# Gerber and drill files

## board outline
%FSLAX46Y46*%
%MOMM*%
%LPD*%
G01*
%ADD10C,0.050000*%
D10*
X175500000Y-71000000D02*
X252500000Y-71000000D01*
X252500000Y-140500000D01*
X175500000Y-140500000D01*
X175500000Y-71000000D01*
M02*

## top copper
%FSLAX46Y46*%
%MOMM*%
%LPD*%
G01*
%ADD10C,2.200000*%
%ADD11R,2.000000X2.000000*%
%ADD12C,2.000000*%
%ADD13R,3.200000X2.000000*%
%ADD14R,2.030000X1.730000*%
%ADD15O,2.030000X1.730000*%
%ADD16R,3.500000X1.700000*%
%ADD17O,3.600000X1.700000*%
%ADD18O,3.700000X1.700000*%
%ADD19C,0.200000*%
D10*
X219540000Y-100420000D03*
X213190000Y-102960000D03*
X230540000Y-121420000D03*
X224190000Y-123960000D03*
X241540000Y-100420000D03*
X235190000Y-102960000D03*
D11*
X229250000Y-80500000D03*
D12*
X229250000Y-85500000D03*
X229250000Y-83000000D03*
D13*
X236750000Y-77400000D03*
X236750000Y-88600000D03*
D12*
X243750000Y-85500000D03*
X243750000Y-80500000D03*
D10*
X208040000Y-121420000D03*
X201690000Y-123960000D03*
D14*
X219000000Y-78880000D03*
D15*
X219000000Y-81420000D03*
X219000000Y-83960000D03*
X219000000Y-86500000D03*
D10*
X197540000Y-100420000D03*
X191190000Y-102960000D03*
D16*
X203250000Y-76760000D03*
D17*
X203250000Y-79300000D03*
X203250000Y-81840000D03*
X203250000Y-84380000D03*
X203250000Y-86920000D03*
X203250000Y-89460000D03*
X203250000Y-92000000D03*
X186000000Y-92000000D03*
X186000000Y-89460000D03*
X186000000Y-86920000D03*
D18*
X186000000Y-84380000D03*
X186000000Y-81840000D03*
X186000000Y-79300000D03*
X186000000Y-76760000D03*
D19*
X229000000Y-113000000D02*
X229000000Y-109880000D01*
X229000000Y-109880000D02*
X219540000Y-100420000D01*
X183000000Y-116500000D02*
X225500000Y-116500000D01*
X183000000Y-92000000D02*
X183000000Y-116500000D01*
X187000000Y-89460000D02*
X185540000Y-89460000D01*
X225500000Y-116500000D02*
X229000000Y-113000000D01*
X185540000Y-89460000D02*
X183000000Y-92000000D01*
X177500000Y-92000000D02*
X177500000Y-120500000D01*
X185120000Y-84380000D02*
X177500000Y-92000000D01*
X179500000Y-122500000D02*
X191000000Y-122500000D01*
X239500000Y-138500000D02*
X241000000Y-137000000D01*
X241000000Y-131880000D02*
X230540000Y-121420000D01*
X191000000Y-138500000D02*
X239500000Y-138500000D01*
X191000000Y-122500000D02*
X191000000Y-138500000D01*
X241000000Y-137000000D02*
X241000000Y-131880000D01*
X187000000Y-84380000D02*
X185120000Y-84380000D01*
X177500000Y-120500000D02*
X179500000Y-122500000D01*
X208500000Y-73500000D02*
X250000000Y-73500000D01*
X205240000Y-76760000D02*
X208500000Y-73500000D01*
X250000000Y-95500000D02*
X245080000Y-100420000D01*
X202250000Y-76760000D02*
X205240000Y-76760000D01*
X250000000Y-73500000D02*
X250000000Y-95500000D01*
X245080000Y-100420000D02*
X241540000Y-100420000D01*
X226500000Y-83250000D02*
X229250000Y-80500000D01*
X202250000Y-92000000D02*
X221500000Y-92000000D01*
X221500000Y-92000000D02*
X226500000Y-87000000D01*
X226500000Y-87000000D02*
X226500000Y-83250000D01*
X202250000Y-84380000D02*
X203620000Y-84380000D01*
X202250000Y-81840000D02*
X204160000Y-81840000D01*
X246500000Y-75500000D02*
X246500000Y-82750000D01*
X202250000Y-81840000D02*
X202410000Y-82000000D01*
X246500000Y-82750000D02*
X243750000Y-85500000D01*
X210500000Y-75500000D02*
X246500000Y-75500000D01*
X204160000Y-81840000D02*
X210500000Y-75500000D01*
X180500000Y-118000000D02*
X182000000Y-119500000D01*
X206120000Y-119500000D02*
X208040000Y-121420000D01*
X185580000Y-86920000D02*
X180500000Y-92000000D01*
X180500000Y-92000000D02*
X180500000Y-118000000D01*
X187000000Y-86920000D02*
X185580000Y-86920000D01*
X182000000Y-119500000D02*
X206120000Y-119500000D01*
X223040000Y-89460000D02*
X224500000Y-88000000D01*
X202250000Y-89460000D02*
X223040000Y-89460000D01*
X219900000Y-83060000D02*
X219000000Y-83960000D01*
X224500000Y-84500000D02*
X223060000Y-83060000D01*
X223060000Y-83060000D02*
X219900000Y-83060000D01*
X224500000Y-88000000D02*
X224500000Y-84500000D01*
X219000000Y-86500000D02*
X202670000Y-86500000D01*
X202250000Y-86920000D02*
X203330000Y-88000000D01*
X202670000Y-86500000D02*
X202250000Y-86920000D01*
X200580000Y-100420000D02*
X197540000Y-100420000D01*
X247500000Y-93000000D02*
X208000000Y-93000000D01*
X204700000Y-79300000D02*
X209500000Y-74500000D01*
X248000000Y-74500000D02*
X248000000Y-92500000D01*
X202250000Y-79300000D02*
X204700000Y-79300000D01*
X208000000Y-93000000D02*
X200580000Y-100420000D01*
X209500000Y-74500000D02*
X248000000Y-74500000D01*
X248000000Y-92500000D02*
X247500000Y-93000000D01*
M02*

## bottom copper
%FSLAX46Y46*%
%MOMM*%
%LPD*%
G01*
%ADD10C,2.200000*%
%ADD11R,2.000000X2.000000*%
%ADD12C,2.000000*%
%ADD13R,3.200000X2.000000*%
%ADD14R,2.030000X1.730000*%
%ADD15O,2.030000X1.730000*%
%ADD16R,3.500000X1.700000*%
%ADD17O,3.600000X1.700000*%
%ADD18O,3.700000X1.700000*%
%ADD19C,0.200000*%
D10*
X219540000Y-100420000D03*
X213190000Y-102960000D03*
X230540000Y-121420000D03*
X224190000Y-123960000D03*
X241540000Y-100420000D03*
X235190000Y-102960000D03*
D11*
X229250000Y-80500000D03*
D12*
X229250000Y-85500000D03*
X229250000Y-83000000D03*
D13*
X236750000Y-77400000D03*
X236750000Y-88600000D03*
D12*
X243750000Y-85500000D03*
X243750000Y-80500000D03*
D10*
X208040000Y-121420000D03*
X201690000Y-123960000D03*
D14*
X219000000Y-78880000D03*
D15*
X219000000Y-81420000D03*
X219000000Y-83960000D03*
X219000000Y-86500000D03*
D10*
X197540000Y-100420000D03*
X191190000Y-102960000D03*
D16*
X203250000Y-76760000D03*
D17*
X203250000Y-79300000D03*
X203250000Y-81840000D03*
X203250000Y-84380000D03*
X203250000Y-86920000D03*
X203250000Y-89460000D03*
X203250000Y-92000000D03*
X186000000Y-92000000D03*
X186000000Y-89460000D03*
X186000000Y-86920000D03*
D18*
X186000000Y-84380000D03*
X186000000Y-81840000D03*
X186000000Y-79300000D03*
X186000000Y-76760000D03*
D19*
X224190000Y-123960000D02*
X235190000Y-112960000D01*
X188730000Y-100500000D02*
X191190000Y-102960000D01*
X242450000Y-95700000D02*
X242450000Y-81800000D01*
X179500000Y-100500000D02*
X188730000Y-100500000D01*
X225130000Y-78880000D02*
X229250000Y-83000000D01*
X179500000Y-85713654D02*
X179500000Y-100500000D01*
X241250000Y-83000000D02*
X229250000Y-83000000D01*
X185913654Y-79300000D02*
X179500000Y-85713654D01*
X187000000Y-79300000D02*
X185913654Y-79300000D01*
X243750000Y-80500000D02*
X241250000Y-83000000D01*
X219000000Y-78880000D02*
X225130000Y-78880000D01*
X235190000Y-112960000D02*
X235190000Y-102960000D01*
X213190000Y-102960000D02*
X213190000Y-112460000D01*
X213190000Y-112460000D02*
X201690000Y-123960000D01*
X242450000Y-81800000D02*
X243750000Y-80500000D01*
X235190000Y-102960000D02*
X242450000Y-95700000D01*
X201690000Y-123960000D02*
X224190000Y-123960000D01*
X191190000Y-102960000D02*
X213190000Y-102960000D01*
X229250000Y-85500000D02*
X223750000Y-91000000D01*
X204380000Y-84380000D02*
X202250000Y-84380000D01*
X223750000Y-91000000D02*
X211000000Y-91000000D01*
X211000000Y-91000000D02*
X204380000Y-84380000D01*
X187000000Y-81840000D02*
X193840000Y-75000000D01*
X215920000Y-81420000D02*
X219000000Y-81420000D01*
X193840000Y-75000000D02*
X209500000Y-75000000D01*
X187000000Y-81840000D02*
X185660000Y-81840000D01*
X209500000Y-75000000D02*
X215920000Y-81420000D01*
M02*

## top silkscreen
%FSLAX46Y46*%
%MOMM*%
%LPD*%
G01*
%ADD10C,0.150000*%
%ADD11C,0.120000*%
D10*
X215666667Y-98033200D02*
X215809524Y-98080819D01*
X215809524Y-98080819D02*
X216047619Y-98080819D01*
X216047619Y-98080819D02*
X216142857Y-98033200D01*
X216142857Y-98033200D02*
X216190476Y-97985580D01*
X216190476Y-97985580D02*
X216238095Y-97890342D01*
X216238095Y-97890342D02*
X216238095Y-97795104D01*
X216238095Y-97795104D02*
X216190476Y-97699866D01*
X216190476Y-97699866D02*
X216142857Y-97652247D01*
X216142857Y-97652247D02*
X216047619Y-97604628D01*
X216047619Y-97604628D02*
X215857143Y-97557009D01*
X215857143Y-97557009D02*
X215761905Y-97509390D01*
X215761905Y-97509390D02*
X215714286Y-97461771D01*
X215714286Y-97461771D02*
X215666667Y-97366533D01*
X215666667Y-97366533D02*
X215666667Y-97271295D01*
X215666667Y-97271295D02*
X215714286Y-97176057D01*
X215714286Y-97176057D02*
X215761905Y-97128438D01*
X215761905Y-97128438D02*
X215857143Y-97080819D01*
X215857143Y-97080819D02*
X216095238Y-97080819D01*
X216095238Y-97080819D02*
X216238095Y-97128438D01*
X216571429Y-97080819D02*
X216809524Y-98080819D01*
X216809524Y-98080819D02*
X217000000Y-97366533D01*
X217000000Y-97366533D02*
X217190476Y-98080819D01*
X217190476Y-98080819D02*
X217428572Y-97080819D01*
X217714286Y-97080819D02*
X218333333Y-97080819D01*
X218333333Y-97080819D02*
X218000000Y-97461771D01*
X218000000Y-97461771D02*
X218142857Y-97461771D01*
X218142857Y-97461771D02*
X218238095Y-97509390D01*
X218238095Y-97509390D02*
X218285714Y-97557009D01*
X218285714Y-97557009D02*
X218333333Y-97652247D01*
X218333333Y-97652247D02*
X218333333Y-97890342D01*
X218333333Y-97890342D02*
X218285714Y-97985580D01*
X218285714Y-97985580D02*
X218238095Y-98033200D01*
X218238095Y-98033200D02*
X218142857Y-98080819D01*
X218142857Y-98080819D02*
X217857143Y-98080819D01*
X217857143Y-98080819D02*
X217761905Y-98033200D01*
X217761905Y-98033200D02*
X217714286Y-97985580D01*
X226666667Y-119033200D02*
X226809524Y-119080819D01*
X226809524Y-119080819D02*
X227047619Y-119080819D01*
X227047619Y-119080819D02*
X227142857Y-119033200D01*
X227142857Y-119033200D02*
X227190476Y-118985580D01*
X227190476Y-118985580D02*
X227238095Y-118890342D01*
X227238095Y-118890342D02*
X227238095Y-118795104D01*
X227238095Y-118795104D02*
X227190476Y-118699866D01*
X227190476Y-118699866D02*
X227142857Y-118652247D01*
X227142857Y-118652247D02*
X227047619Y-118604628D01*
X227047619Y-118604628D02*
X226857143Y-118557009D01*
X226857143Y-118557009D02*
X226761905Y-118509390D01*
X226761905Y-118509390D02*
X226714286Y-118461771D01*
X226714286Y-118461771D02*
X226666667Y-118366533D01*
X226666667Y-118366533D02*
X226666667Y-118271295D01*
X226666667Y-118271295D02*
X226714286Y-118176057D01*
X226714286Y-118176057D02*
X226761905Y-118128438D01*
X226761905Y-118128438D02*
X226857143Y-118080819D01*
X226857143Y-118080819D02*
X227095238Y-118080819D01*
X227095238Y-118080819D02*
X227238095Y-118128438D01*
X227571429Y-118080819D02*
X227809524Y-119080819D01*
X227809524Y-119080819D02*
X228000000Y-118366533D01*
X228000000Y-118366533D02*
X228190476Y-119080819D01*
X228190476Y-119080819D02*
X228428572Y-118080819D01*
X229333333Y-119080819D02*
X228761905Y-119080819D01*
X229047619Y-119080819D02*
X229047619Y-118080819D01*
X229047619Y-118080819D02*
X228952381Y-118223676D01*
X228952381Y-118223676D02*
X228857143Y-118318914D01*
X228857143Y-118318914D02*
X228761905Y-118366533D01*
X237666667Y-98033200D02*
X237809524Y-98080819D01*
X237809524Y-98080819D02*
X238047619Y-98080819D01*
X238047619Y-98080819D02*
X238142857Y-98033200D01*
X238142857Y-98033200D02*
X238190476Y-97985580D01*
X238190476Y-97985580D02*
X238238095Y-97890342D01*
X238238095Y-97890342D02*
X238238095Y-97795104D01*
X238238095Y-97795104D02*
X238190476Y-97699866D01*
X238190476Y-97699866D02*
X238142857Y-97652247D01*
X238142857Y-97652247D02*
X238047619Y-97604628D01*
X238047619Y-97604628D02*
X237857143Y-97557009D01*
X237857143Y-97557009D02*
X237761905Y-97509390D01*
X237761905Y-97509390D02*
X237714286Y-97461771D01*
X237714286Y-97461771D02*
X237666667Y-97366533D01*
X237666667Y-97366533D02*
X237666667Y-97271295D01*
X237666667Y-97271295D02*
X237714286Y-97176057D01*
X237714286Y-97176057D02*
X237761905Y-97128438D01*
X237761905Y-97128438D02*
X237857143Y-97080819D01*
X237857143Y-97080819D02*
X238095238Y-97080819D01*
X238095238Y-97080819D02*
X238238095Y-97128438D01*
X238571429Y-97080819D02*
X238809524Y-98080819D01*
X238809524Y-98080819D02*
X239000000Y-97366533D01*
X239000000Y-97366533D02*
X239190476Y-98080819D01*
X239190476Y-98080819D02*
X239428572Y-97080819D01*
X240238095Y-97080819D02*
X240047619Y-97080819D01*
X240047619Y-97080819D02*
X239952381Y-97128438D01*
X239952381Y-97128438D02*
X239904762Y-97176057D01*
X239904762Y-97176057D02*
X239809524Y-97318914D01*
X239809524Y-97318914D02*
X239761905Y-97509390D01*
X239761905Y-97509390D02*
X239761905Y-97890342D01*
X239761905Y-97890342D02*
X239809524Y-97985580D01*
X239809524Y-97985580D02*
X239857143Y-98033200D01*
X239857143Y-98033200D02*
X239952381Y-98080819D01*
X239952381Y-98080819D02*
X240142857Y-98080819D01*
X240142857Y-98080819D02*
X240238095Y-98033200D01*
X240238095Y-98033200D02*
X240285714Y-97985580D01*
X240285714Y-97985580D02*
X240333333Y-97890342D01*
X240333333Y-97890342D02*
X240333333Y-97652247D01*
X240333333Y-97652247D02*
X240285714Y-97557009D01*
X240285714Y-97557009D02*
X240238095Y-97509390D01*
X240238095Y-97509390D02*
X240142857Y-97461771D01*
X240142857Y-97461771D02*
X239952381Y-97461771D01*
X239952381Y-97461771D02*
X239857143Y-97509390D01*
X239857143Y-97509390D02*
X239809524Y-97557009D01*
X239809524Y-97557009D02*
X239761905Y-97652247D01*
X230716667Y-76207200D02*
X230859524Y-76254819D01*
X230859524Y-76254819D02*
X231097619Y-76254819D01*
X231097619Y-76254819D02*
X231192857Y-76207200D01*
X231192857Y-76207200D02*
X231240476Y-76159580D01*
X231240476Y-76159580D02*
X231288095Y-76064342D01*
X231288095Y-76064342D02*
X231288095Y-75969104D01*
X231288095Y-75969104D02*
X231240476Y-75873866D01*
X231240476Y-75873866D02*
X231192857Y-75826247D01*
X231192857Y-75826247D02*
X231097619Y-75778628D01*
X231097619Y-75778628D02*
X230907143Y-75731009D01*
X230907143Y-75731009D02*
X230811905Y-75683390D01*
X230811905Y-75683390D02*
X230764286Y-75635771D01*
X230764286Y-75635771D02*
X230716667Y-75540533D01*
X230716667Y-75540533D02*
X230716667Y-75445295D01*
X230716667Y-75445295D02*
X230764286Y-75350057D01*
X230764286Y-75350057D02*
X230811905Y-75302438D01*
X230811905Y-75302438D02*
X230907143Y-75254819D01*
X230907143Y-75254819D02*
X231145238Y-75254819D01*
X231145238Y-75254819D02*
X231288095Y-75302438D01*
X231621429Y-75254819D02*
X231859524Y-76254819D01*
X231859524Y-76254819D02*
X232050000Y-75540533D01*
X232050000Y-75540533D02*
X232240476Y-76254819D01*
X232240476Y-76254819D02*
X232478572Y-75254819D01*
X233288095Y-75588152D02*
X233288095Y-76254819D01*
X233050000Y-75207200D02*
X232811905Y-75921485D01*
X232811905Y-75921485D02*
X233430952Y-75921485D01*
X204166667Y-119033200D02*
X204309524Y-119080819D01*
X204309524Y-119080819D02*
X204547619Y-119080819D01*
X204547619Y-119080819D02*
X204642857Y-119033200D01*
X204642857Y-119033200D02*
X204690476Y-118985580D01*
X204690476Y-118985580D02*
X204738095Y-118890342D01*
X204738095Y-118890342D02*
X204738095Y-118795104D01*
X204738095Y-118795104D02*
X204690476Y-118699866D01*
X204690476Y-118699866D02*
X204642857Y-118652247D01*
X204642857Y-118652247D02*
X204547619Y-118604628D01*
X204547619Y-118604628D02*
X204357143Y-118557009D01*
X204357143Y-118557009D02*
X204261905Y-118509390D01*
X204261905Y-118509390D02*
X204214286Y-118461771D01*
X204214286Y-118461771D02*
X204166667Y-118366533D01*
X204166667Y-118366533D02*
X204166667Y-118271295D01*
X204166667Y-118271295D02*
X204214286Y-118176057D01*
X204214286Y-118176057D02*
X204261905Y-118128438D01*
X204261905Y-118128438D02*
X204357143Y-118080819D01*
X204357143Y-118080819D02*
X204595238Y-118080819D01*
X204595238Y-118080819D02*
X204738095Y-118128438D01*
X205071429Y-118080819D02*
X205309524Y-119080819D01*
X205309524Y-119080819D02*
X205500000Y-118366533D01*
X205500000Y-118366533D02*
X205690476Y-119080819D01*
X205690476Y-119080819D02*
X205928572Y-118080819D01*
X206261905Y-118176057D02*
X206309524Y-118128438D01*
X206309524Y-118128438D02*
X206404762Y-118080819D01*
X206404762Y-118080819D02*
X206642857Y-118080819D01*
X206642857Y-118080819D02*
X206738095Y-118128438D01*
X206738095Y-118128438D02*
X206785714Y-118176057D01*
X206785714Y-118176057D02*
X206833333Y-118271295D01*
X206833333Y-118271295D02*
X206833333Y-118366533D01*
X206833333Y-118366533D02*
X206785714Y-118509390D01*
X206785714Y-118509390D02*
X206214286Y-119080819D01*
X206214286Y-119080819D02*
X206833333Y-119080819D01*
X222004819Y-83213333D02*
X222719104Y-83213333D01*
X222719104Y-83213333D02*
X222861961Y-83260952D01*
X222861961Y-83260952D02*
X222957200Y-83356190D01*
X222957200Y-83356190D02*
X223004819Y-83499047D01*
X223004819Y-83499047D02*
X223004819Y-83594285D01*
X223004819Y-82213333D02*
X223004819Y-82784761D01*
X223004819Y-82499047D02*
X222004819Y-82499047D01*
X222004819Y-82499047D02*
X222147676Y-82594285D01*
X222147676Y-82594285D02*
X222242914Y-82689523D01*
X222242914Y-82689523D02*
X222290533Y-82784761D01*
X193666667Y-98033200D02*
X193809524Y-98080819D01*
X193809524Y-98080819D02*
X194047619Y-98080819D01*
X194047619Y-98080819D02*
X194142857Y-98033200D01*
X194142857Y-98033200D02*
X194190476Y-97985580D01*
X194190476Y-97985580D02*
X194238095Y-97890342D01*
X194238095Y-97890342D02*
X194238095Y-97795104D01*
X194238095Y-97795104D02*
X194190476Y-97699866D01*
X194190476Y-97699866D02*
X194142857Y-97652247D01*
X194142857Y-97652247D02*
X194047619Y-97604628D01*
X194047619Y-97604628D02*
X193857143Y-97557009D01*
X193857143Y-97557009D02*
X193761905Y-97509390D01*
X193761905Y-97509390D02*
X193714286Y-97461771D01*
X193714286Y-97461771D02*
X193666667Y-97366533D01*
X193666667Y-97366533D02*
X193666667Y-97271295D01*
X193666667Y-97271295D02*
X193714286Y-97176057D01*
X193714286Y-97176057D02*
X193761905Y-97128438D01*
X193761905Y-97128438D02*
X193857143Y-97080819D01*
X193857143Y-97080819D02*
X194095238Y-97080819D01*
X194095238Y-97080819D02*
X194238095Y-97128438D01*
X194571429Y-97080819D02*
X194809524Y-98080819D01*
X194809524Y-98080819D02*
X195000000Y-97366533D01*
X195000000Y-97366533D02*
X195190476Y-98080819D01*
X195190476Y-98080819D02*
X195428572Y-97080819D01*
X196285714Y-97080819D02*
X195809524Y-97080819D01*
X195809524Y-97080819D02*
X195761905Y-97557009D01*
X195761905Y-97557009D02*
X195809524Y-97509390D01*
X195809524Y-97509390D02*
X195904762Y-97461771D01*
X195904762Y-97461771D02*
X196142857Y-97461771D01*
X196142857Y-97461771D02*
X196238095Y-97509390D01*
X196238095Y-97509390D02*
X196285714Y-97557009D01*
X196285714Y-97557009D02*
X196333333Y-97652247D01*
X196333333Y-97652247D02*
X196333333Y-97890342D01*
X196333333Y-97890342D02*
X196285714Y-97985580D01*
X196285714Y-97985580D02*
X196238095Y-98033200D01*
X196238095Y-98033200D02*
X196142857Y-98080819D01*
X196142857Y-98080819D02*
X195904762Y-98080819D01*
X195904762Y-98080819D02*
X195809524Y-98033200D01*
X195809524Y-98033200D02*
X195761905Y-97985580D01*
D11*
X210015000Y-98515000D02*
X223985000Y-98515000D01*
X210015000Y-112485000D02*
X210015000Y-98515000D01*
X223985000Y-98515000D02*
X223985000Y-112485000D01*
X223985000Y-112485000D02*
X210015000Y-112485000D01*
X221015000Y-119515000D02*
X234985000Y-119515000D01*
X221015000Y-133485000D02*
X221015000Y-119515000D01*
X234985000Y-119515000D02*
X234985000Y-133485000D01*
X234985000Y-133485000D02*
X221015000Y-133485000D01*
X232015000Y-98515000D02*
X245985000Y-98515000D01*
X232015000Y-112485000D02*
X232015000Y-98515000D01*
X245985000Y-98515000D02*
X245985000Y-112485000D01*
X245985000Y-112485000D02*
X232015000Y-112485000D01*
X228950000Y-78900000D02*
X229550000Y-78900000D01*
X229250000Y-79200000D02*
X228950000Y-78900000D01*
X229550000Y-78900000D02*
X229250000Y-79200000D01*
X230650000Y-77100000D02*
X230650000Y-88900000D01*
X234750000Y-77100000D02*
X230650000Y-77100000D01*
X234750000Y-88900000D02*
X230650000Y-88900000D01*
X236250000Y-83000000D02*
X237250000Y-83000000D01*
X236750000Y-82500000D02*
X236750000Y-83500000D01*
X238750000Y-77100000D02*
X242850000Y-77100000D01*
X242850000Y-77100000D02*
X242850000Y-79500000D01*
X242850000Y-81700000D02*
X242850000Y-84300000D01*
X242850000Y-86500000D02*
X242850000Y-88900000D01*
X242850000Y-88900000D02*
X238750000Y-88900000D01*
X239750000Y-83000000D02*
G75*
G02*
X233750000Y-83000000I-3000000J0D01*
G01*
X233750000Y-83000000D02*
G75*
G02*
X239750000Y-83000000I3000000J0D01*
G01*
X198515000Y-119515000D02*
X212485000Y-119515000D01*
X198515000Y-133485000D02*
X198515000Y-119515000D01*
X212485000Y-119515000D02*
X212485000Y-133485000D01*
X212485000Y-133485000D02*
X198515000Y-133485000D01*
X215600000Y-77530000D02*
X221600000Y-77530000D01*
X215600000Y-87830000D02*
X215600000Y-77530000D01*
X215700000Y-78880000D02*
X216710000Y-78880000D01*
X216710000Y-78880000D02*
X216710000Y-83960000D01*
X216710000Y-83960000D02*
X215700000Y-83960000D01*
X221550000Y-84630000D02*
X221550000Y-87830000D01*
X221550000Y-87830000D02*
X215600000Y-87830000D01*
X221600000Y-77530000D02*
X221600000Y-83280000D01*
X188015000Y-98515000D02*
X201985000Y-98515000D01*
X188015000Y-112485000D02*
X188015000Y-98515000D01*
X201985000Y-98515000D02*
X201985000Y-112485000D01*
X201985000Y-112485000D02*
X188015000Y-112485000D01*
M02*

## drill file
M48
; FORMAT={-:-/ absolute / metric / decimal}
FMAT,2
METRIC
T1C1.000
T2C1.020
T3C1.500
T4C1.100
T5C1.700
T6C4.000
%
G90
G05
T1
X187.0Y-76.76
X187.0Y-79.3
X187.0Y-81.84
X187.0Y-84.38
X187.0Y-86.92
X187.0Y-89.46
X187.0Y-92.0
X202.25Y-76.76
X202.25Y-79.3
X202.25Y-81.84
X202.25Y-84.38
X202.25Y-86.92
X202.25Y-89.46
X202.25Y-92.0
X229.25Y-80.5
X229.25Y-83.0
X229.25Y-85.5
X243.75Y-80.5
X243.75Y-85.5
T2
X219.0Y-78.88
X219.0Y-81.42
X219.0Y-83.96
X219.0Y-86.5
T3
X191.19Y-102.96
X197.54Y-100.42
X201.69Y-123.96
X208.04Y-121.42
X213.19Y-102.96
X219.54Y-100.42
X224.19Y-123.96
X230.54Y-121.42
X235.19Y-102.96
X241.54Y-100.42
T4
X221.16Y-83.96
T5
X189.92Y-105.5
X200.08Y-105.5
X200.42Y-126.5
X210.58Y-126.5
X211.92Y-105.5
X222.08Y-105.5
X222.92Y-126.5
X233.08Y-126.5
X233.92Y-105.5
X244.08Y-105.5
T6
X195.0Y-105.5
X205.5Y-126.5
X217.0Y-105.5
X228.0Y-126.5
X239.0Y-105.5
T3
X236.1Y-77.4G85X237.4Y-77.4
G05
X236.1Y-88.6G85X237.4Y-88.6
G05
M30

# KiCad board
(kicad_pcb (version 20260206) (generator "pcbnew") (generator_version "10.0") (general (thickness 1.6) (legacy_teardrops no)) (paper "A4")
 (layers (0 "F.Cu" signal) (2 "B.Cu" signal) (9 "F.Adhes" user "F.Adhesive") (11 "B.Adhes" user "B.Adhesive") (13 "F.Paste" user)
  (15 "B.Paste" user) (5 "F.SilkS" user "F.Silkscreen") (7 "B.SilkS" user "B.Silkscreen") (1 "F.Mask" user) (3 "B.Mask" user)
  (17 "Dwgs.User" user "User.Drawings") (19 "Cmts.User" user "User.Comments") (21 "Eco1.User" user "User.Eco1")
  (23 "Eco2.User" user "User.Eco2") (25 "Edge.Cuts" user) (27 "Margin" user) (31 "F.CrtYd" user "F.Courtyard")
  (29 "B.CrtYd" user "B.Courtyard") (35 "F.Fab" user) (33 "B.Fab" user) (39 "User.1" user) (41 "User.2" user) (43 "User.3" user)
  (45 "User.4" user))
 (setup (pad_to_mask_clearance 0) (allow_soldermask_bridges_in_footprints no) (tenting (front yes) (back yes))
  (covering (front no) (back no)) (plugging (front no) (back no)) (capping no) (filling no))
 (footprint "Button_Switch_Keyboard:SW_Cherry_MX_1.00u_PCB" (layer "F.Cu") (at 219.54 100.42)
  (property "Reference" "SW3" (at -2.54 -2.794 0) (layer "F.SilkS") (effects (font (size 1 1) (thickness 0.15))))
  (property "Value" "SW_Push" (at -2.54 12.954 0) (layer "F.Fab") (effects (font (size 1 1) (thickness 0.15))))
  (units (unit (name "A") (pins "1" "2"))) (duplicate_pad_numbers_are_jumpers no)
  (fp_line (start -9.525 -1.905) (end 4.445 -1.905) (stroke (width 0.12) (type solid)) (layer "F.SilkS"))
  (fp_line (start -9.525 12.065) (end -9.525 -1.905) (stroke (width 0.12) (type solid)) (layer "F.SilkS"))
  (fp_line (start 4.445 -1.905) (end 4.445 12.065) (stroke (width 0.12) (type solid)) (layer "F.SilkS"))
  (fp_line (start 4.445 12.065) (end -9.525 12.065) (stroke (width 0.12) (type solid)) (layer "F.SilkS"))
  (pad "" np_thru_hole circle (at -7.62 5.08) (size 1.7 1.7) (drill 1.7) (layers "*.Cu" "*.Mask"))
  (pad "" np_thru_hole circle (at -2.54 5.08) (size 4 4) (drill 4) (layers "*.Cu" "*.Mask"))
  (pad "" np_thru_hole circle (at 2.54 5.08) (size 1.7 1.7) (drill 1.7) (layers "*.Cu" "*.Mask"))
  (pad "1" thru_hole circle (at 0 0) (size 2.2 2.2) (drill 1.5) (layers "*.Cu" "*.Mask") (remove_unused_layers no)
   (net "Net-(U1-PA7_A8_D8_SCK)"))
  (pad "2" thru_hole circle (at -6.35 2.54) (size 2.2 2.2) (drill 1.5) (layers "*.Cu" "*.Mask") (remove_unused_layers no) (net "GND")))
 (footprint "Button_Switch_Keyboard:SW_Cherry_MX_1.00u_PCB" (layer "F.Cu") (at 230.54 121.42)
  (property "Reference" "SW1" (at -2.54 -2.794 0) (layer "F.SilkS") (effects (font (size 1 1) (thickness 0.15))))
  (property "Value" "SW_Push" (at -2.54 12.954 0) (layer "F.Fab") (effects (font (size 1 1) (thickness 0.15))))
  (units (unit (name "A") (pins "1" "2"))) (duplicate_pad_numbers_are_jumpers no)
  (fp_line (start -9.525 -1.905) (end 4.445 -1.905) (stroke (width 0.12) (type solid)) (layer "F.SilkS"))
  (fp_line (start -9.525 12.065) (end -9.525 -1.905) (stroke (width 0.12) (type solid)) (layer "F.SilkS"))
  (fp_line (start 4.445 -1.905) (end 4.445 12.065) (stroke (width 0.12) (type solid)) (layer "F.SilkS"))
  (fp_line (start 4.445 12.065) (end -9.525 12.065) (stroke (width 0.12) (type solid)) (layer "F.SilkS"))
  (pad "" np_thru_hole circle (at -7.62 5.08) (size 1.7 1.7) (drill 1.7) (layers "*.Cu" "*.Mask"))
  (pad "" np_thru_hole circle (at -2.54 5.08) (size 4 4) (drill 4) (layers "*.Cu" "*.Mask"))
  (pad "" np_thru_hole circle (at 2.54 5.08) (size 1.7 1.7) (drill 1.7) (layers "*.Cu" "*.Mask"))
  (pad "1" thru_hole circle (at 0 0) (size 2.2 2.2) (drill 1.5) (layers "*.Cu" "*.Mask") (remove_unused_layers no)
   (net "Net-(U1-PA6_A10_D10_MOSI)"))
  (pad "2" thru_hole circle (at -6.35 2.54) (size 2.2 2.2) (drill 1.5) (layers "*.Cu" "*.Mask") (remove_unused_layers no) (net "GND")))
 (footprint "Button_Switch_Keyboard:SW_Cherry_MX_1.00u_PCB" (layer "F.Cu") (at 241.54 100.42)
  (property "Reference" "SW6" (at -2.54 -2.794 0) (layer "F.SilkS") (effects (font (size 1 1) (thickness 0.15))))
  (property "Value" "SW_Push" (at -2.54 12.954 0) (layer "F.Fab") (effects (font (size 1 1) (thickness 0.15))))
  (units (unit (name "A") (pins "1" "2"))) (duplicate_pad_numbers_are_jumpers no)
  (fp_line (start -9.525 -1.905) (end 4.445 -1.905) (stroke (width 0.12) (type solid)) (layer "F.SilkS"))
  (fp_line (start -9.525 12.065) (end -9.525 -1.905) (stroke (width 0.12) (type solid)) (layer "F.SilkS"))
  (fp_line (start 4.445 -1.905) (end 4.445 12.065) (stroke (width 0.12) (type solid)) (layer "F.SilkS"))
  (fp_line (start 4.445 12.065) (end -9.525 12.065) (stroke (width 0.12) (type solid)) (layer "F.SilkS"))
  (pad "" np_thru_hole circle (at -7.62 5.08) (size 1.7 1.7) (drill 1.7) (layers "*.Cu" "*.Mask"))
  (pad "" np_thru_hole circle (at -2.54 5.08) (size 4 4) (drill 4) (layers "*.Cu" "*.Mask"))
  (pad "" np_thru_hole circle (at 2.54 5.08) (size 1.7 1.7) (drill 1.7) (layers "*.Cu" "*.Mask"))
  (pad "1" thru_hole circle (at 0 0) (size 2.2 2.2) (drill 1.5) (layers "*.Cu" "*.Mask") (remove_unused_layers no)
   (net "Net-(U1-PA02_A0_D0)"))
  (pad "2" thru_hole circle (at -6.35 2.54) (size 2.2 2.2) (drill 1.5) (layers "*.Cu" "*.Mask") (remove_unused_layers no) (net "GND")))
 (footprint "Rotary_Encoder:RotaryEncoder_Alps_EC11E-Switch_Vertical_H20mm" (layer "F.Cu") (at 229.25 80.5)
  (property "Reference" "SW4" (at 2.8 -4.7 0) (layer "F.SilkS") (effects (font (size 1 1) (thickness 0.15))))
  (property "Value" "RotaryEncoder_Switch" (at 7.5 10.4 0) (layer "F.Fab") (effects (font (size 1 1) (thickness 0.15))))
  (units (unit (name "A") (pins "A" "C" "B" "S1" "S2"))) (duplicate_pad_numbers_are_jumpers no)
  (fp_line (start -0.3 -1.6) (end 0.3 -1.6) (stroke (width 0.12) (type solid)) (layer "F.SilkS"))
  (fp_line (start 0 -1.3) (end -0.3 -1.6) (stroke (width 0.12) (type solid)) (layer "F.SilkS"))
  (fp_line (start 0.3 -1.6) (end 0 -1.3) (stroke (width 0.12) (type solid)) (layer "F.SilkS"))
  (fp_line (start 1.4 -3.4) (end 1.4 8.4) (stroke (width 0.12) (type solid)) (layer "F.SilkS"))
  (fp_line (start 5.5 -3.4) (end 1.4 -3.4) (stroke (width 0.12) (type solid)) (layer "F.SilkS"))
  (fp_line (start 5.5 8.4) (end 1.4 8.4) (stroke (width 0.12) (type solid)) (layer "F.SilkS"))
  (fp_line (start 7 2.5) (end 8 2.5) (stroke (width 0.12) (type solid)) (layer "F.SilkS"))
  (fp_line (start 7.5 2) (end 7.5 3) (stroke (width 0.12) (type solid)) (layer "F.SilkS"))
  (fp_line (start 9.5 -3.4) (end 13.6 -3.4) (stroke (width 0.12) (type solid)) (layer "F.SilkS"))
  (fp_line (start 13.6 -3.4) (end 13.6 -1) (stroke (width 0.12) (type solid)) (layer "F.SilkS"))
  (fp_line (start 13.6 1.2) (end 13.6 3.8) (stroke (width 0.12) (type solid)) (layer "F.SilkS"))
  (fp_line (start 13.6 6) (end 13.6 8.4) (stroke (width 0.12) (type solid)) (layer "F.SilkS"))
  (fp_line (start 13.6 8.4) (end 9.5 8.4) (stroke (width 0.12) (type solid)) (layer "F.SilkS"))
  (fp_circle (center 7.5 2.5) (end 10.5 2.5) (stroke (width 0.12) (type solid)) (fill no) (layer "F.SilkS"))
  (pad "A" thru_hole rect (at 0 0) (size 2 2) (drill 1) (layers "*.Cu" "*.Mask") (remove_unused_layers no) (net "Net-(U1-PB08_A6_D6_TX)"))
  (pad "B" thru_hole circle (at 0 5) (size 2 2) (drill 1) (layers "*.Cu" "*.Mask") (remove_unused_layers no) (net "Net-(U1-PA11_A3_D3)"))
  (pad "C" thru_hole circle (at 0 2.5) (size 2 2) (drill 1) (layers "*.Cu" "*.Mask") (remove_unused_layers no) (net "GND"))
  (pad "MP" thru_hole rect (at 7.5 -3.1) (size 3.2 2) (drill oval 2.8 1.5) (layers "*.Cu" "*.Mask") (remove_unused_layers no))
  (pad "MP" thru_hole rect (at 7.5 8.1) (size 3.2 2) (drill oval 2.8 1.5) (layers "*.Cu" "*.Mask") (remove_unused_layers no))
  (pad "S1" thru_hole circle (at 14.5 5) (size 2 2) (drill 1) (layers "*.Cu" "*.Mask") (remove_unused_layers no) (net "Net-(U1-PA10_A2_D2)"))
  (pad "S2" thru_hole circle (at 14.5 0) (size 2 2) (drill 1) (layers "*.Cu" "*.Mask") (remove_unused_layers no) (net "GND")))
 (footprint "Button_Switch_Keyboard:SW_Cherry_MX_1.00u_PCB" (layer "F.Cu") (at 208.04 121.42)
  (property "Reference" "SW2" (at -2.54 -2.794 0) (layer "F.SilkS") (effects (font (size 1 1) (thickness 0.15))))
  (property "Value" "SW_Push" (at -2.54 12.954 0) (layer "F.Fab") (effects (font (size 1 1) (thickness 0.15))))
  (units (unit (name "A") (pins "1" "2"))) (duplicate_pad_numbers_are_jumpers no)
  (fp_line (start -9.525 -1.905) (end 4.445 -1.905) (stroke (width 0.12) (type solid)) (layer "F.SilkS"))
  (fp_line (start -9.525 12.065) (end -9.525 -1.905) (stroke (width 0.12) (type solid)) (layer "F.SilkS"))
  (fp_line (start 4.445 -1.905) (end 4.445 12.065) (stroke (width 0.12) (type solid)) (layer "F.SilkS"))
  (fp_line (start 4.445 12.065) (end -9.525 12.065) (stroke (width 0.12) (type solid)) (layer "F.SilkS"))
  (pad "" np_thru_hole circle (at -7.62 5.08) (size 1.7 1.7) (drill 1.7) (layers "*.Cu" "*.Mask"))
  (pad "" np_thru_hole circle (at -2.54 5.08) (size 4 4) (drill 4) (layers "*.Cu" "*.Mask"))
  (pad "" np_thru_hole circle (at 2.54 5.08) (size 1.7 1.7) (drill 1.7) (layers "*.Cu" "*.Mask"))
  (pad "1" thru_hole circle (at 0 0) (size 2.2 2.2) (drill 1.5) (layers "*.Cu" "*.Mask") (remove_unused_layers no)
   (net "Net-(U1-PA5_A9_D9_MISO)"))
  (pad "2" thru_hole circle (at -6.35 2.54) (size 2.2 2.2) (drill 1.5) (layers "*.Cu" "*.Mask") (remove_unused_layers no) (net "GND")))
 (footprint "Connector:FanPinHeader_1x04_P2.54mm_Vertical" (layer "F.Cu") (at 219 78.88 -90)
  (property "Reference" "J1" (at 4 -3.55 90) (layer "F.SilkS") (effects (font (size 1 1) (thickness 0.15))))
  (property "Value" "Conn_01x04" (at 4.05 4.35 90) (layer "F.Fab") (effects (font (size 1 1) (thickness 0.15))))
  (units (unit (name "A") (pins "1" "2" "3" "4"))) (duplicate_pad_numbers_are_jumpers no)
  (fp_line (start -1.35 3.4) (end -1.35 -2.6) (stroke (width 0.12) (type solid)) (layer "F.SilkS"))
  (fp_line (start 8.95 3.4) (end -1.35 3.4) (stroke (width 0.12) (type solid)) (layer "F.SilkS"))
  (fp_line (start 0 3.3) (end 0 2.29) (stroke (width 0.12) (type solid)) (layer "F.SilkS"))
  (fp_line (start 0 2.29) (end 5.08 2.29) (stroke (width 0.12) (type solid)) (layer "F.SilkS"))
  (fp_line (start 5.08 2.29) (end 5.08 3.3) (stroke (width 0.12) (type solid)) (layer "F.SilkS"))
  (fp_line (start 5.75 -2.55) (end 8.95 -2.55) (stroke (width 0.12) (type solid)) (layer "F.SilkS"))
  (fp_line (start 8.95 -2.55) (end 8.95 3.4) (stroke (width 0.12) (type solid)) (layer "F.SilkS"))
  (fp_line (start -1.35 -2.6) (end 4.4 -2.6) (stroke (width 0.12) (type solid)) (layer "F.SilkS"))
  (pad "" np_thru_hole circle (at 5.08 -2.16) (size 1.1 1.1) (drill 1.1) (layers "*.Cu" "*.Mask"))
  (pad "1" thru_hole rect (at 0 0) (size 2.03 1.73) (drill 1.02) (layers "*.Cu" "*.Mask") (remove_unused_layers no) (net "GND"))
  (pad "2" thru_hole oval (at 2.54 0) (size 2.03 1.73) (drill 1.02) (layers "*.Cu" "*.Mask") (remove_unused_layers no) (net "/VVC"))
  (pad "3" thru_hole oval (at 5.08 0) (size 2.03 1.73) (drill 1.02) (layers "*.Cu" "*.Mask") (remove_unused_layers no) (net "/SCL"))
  (pad "4" thru_hole oval (at 7.62 0) (size 2.03 1.73) (drill 1.02) (layers "*.Cu" "*.Mask") (remove_unused_layers no) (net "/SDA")))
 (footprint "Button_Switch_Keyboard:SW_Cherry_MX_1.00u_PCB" (layer "F.Cu") (at 197.54 100.42)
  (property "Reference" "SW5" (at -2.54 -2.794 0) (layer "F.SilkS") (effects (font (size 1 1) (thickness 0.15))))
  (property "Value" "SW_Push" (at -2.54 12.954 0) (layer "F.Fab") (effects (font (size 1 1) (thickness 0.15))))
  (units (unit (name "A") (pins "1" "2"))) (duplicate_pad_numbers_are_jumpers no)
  (fp_line (start -9.525 -1.905) (end 4.445 -1.905) (stroke (width 0.12) (type solid)) (layer "F.SilkS"))
  (fp_line (start -9.525 12.065) (end -9.525 -1.905) (stroke (width 0.12) (type solid)) (layer "F.SilkS"))
  (fp_line (start 4.445 -1.905) (end 4.445 12.065) (stroke (width 0.12) (type solid)) (layer "F.SilkS"))
  (fp_line (start 4.445 12.065) (end -9.525 12.065) (stroke (width 0.12) (type solid)) (layer "F.SilkS"))
  (pad "" np_thru_hole circle (at -7.62 5.08) (size 1.7 1.7) (drill 1.7) (layers "*.Cu" "*.Mask"))
  (pad "" np_thru_hole circle (at -2.54 5.08) (size 4 4) (drill 4) (layers "*.Cu" "*.Mask"))
  (pad "" np_thru_hole circle (at 2.54 5.08) (size 1.7 1.7) (drill 1.7) (layers "*.Cu" "*.Mask"))
  (pad "1" thru_hole circle (at 0 0) (size 2.2 2.2) (drill 1.5) (layers "*.Cu" "*.Mask") (remove_unused_layers no)
   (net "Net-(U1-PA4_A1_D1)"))
  (pad "2" thru_hole circle (at -6.35 2.54) (size 2.2 2.2) (drill 1.5) (layers "*.Cu" "*.Mask") (remove_unused_layers no) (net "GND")))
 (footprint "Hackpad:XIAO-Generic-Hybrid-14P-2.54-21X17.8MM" (layer "B.Cu") (at 194.625 84.38 180)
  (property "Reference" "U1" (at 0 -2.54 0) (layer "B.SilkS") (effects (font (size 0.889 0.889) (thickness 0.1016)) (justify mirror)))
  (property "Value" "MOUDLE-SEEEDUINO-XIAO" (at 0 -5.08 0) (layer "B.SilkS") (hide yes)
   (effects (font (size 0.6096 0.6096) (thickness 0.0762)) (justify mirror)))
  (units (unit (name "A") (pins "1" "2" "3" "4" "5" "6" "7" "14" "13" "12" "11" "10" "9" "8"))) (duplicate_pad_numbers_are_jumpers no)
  (pad "1" thru_hole rect (at -7.625 7.62 180) (size 3.5 1.7) (drill 1 (offset -1 0)) (layers "*.Cu" "*.Mask") (remove_unused_layers no)
   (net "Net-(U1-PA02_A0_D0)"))
  (pad "2" thru_hole oval (at -7.625 5.08 180) (size 3.6 1.7) (drill 1 (offset -1 0)) (layers "*.Cu" "*.Mask") (remove_unused_layers no)
   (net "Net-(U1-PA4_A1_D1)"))
  (pad "3" thru_hole oval (at -7.625 2.54 180) (size 3.6 1.7) (drill 1 (offset -1 0)) (layers "*.Cu" "*.Mask") (remove_unused_layers no)
   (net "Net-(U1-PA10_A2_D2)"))
  (pad "4" thru_hole oval (at -7.625 0 180) (size 3.6 1.7) (drill 1 (offset -1 0)) (layers "*.Cu" "*.Mask") (remove_unused_layers no)
   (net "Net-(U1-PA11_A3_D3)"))
  (pad "5" thru_hole oval (at -7.625 -2.54 180) (size 3.6 1.7) (drill 1 (offset -1 0)) (layers "*.Cu" "*.Mask") (remove_unused_layers no)
   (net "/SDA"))
  (pad "6" thru_hole oval (at -7.625 -5.08) (size 3.6 1.7) (drill 1 (offset 1 0)) (layers "*.Cu" "*.Mask") (remove_unused_layers no)
   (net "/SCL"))
  (pad "7" thru_hole oval (at -7.625 -7.62 180) (size 3.6 1.7) (drill 1 (offset -1 0)) (layers "*.Cu" "*.Mask") (remove_unused_layers no)
   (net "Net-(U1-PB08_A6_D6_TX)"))
  (pad "8" thru_hole oval (at 7.625 -7.62 180) (size 3.6 1.7) (drill 1 (offset 1 0)) (layers "*.Cu" "*.Mask") (remove_unused_layers no)
   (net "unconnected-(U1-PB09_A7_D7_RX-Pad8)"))
  (pad "9" thru_hole oval (at 7.625 -5.08 180) (size 3.6 1.7) (drill 1 (offset 1 0)) (layers "*.Cu" "*.Mask") (remove_unused_layers no)
   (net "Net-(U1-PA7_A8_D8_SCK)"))
  (pad "10" thru_hole oval (at 7.625 -2.54 180) (size 3.6 1.7) (drill 1 (offset 1 0)) (layers "*.Cu" "*.Mask") (remove_unused_layers no)
   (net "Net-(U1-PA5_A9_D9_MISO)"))
  (pad "11" thru_hole oval (at 7.625 0 180) (size 3.7 1.7) (drill 1 (offset 1 0)) (layers "*.Cu" "*.Mask") (remove_unused_layers no)
   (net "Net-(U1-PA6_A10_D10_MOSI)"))
  (pad "12" thru_hole oval (at 7.625 2.54 180) (size 3.7 1.7) (drill 1 (offset 1 0)) (layers "*.Cu" "*.Mask") (remove_unused_layers no)
   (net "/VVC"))
  (pad "13" thru_hole oval (at 7.625 5.08 180) (size 3.7 1.7) (drill 1 (offset 1 0)) (layers "*.Cu" "*.Mask") (remove_unused_layers no)
   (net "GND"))
  (pad "14" thru_hole oval (at 7.625 7.62 180) (size 3.7 1.7) (drill 1 (offset 1 0)) (layers "*.Cu" "*.Mask") (remove_unused_layers no)
   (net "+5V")))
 (gr_rect (start 175.5 71) (end 252.5 140.5) (stroke (width 0.05) (type default)) (fill no) (layer "Edge.Cuts"))
 (segment (start 229 113) (end 229 109.88) (width 0.2) (layer "F.Cu") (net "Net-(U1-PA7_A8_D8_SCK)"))
 (segment (start 229 109.88) (end 219.54 100.42) (width 0.2) (layer "F.Cu") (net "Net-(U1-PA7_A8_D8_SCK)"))
 (segment (start 183 116.5) (end 225.5 116.5) (width 0.2) (layer "F.Cu") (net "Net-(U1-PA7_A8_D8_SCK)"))
 (segment (start 183 92) (end 183 116.5) (width 0.2) (layer "F.Cu") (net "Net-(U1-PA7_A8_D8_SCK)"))
 (segment (start 187 89.46) (end 185.54 89.46) (width 0.2) (layer "F.Cu") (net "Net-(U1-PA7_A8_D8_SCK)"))
 (segment (start 225.5 116.5) (end 229 113) (width 0.2) (layer "F.Cu") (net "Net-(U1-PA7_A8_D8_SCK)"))
 (segment (start 185.54 89.46) (end 183 92) (width 0.2) (layer "F.Cu") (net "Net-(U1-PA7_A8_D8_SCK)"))
 (segment (start 224.19 123.96) (end 235.19 112.96) (width 0.2) (layer "B.Cu") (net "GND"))
 (segment (start 188.73 100.5) (end 191.19 102.96) (width 0.2) (layer "B.Cu") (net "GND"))
 (segment (start 242.45 95.7) (end 242.45 81.8) (width 0.2) (layer "B.Cu") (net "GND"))
 (segment (start 179.5 100.5) (end 188.73 100.5) (width 0.2) (layer "B.Cu") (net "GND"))
 (segment (start 225.13 78.88) (end 229.25 83) (width 0.2) (layer "B.Cu") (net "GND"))
 (segment (start 179.5 85.713654) (end 179.5 100.5) (width 0.2) (layer "B.Cu") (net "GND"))
 (segment (start 241.25 83) (end 229.25 83) (width 0.2) (layer "B.Cu") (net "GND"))
 (segment (start 185.913654 79.3) (end 179.5 85.713654) (width 0.2) (layer "B.Cu") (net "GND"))
 (segment (start 187 79.3) (end 185.913654 79.3) (width 0.2) (layer "B.Cu") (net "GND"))
 (segment (start 243.75 80.5) (end 241.25 83) (width 0.2) (layer "B.Cu") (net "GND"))
 (segment (start 219 78.88) (end 225.13 78.88) (width 0.2) (layer "B.Cu") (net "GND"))
 (segment (start 235.19 112.96) (end 235.19 102.96) (width 0.2) (layer "B.Cu") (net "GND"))
 (segment (start 213.19 102.96) (end 213.19 112.46) (width 0.2) (layer "B.Cu") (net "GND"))
 (segment (start 213.19 112.46) (end 201.69 123.96) (width 0.2) (layer "B.Cu") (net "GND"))
 (segment (start 242.45 81.8) (end 243.75 80.5) (width 0.2) (layer "B.Cu") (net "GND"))
 (segment (start 235.19 102.96) (end 242.45 95.7) (width 0.2) (layer "B.Cu") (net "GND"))
 (segment (start 201.69 123.96) (end 224.19 123.96) (width 0.2) (layer "B.Cu") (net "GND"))
 (segment (start 191.19 102.96) (end 213.19 102.96) (width 0.2) (layer "B.Cu") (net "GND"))
 (segment (start 177.5 92) (end 177.5 120.5) (width 0.2) (layer "F.Cu") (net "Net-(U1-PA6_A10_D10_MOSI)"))
 (segment (start 185.12 84.38) (end 177.5 92) (width 0.2) (layer "F.Cu") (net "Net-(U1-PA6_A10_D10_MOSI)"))
 (segment (start 179.5 122.5) (end 191 122.5) (width 0.2) (layer "F.Cu") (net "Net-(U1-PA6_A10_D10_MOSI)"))
 (segment (start 239.5 138.5) (end 241 137) (width 0.2) (layer "F.Cu") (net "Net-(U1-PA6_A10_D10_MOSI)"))
 (segment (start 241 131.88) (end 230.54 121.42) (width 0.2) (layer "F.Cu") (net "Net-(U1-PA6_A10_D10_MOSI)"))
 (segment (start 191 138.5) (end 239.5 138.5) (width 0.2) (layer "F.Cu") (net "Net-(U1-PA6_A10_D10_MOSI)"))
 (segment (start 191 122.5) (end 191 138.5) (width 0.2) (layer "F.Cu") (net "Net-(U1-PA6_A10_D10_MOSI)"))
 (segment (start 241 137) (end 241 131.88) (width 0.2) (layer "F.Cu") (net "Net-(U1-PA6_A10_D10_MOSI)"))
 (segment (start 187 84.38) (end 185.12 84.38) (width 0.2) (layer "F.Cu") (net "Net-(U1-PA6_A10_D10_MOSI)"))
 (segment (start 177.5 120.5) (end 179.5 122.5) (width 0.2) (layer "F.Cu") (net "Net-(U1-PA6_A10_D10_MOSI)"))
 (segment (start 208.5 73.5) (end 250 73.5) (width 0.2) (layer "F.Cu") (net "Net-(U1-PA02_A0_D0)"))
 (segment (start 205.24 76.76) (end 208.5 73.5) (width 0.2) (layer "F.Cu") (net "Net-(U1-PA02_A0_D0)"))
 (segment (start 250 95.5) (end 245.08 100.42) (width 0.2) (layer "F.Cu") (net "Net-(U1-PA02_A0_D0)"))
 (segment (start 202.25 76.76) (end 205.24 76.76) (width 0.2) (layer "F.Cu") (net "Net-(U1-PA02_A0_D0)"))
 (segment (start 250 73.5) (end 250 95.5) (width 0.2) (layer "F.Cu") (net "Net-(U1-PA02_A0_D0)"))
 (segment (start 245.08 100.42) (end 241.54 100.42) (width 0.2) (layer "F.Cu") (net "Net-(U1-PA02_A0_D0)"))
 (segment (start 226.5 83.25) (end 229.25 80.5) (width 0.2) (layer "F.Cu") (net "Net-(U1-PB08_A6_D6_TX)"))
 (segment (start 202.25 92) (end 221.5 92) (width 0.2) (layer "F.Cu") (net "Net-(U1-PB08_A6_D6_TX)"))
 (segment (start 221.5 92) (end 226.5 87) (width 0.2) (layer "F.Cu") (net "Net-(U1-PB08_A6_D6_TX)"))
 (segment (start 226.5 87) (end 226.5 83.25) (width 0.2) (layer "F.Cu") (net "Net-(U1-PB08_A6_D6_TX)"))
 (segment (start 202.25 84.38) (end 203.62 84.38) (width 0.2) (layer "F.Cu") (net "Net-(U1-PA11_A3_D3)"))
 (segment (start 229.25 85.5) (end 223.75 91) (width 0.2) (layer "B.Cu") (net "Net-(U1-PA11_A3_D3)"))
 (segment (start 204.38 84.38) (end 202.25 84.38) (width 0.2) (layer "B.Cu") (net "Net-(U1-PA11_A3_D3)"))
 (segment (start 223.75 91) (end 211 91) (width 0.2) (layer "B.Cu") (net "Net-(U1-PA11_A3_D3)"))
 (segment (start 211 91) (end 204.38 84.38) (width 0.2) (layer "B.Cu") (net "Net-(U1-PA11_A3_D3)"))
 (segment (start 202.25 81.84) (end 204.16 81.84) (width 0.2) (layer "F.Cu") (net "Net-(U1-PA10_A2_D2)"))
 (segment (start 246.5 75.5) (end 246.5 82.75) (width 0.2) (layer "F.Cu") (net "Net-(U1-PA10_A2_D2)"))
 (segment (start 202.25 81.84) (end 202.41 82) (width 0.2) (layer "F.Cu") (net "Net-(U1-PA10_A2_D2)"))
 (segment (start 246.5 82.75) (end 243.75 85.5) (width 0.2) (layer "F.Cu") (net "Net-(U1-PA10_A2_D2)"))
 (segment (start 210.5 75.5) (end 246.5 75.5) (width 0.2) (layer "F.Cu") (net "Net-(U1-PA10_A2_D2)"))
 (segment (start 204.16 81.84) (end 210.5 75.5) (width 0.2) (layer "F.Cu") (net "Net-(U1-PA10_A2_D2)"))
 (segment (start 180.5 118) (end 182 119.5) (width 0.2) (layer "F.Cu") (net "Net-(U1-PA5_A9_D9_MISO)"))
 (segment (start 206.12 119.5) (end 208.04 121.42) (width 0.2) (layer "F.Cu") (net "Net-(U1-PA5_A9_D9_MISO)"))
 (segment (start 185.58 86.92) (end 180.5 92) (width 0.2) (layer "F.Cu") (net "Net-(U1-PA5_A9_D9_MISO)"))
 (segment (start 180.5 92) (end 180.5 118) (width 0.2) (layer "F.Cu") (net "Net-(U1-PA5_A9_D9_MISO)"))
 (segment (start 187 86.92) (end 185.58 86.92) (width 0.2) (layer "F.Cu") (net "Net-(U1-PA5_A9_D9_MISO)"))
 (segment (start 182 119.5) (end 206.12 119.5) (width 0.2) (layer "F.Cu") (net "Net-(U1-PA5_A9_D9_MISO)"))
 (segment (start 187 81.84) (end 193.84 75) (width 0.2) (layer "B.Cu") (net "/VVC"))
 (segment (start 215.92 81.42) (end 219 81.42) (width 0.2) (layer "B.Cu") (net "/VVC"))
 (segment (start 193.84 75) (end 209.5 75) (width 0.2) (layer "B.Cu") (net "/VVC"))
 (segment (start 187 81.84) (end 185.66 81.84) (width 0.2) (layer "B.Cu") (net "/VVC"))
 (segment (start 209.5 75) (end 215.92 81.42) (width 0.2) (layer "B.Cu") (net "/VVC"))
 (segment (start 223.04 89.46) (end 224.5 88) (width 0.2) (layer "F.Cu") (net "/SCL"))
 (segment (start 202.25 89.46) (end 223.04 89.46) (width 0.2) (layer "F.Cu") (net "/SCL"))
 (segment (start 219.9 83.06) (end 219 83.96) (width 0.2) (layer "F.Cu") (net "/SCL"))
 (segment (start 224.5 84.5) (end 223.06 83.06) (width 0.2) (layer "F.Cu") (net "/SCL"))
 (segment (start 223.06 83.06) (end 219.9 83.06) (width 0.2) (layer "F.Cu") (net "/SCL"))
 (segment (start 224.5 88) (end 224.5 84.5) (width 0.2) (layer "F.Cu") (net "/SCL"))
 (segment (start 219 86.5) (end 202.67 86.5) (width 0.2) (layer "F.Cu") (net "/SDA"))
 (segment (start 202.25 86.92) (end 203.33 88) (width 0.2) (layer "F.Cu") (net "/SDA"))
 (segment (start 202.67 86.5) (end 202.25 86.92) (width 0.2) (layer "F.Cu") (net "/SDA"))
 (segment (start 200.58 100.42) (end 197.54 100.42) (width 0.2) (layer "F.Cu") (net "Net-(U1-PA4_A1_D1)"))
 (segment (start 247.5 93) (end 208 93) (width 0.2) (layer "F.Cu") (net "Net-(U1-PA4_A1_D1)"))
 (segment (start 204.7 79.3) (end 209.5 74.5) (width 0.2) (layer "F.Cu") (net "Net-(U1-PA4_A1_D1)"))
 (segment (start 248 74.5) (end 248 92.5) (width 0.2) (layer "F.Cu") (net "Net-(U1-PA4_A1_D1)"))
 (segment (start 202.25 79.3) (end 204.7 79.3) (width 0.2) (layer "F.Cu") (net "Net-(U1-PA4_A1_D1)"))
 (segment (start 208 93) (end 200.58 100.42) (width 0.2) (layer "F.Cu") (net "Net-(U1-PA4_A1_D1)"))
 (segment (start 209.5 74.5) (end 248 74.5) (width 0.2) (layer "F.Cu") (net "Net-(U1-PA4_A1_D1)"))
 (segment (start 248 92.5) (end 247.5 93) (width 0.2) (layer "F.Cu") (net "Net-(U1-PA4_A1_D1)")))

